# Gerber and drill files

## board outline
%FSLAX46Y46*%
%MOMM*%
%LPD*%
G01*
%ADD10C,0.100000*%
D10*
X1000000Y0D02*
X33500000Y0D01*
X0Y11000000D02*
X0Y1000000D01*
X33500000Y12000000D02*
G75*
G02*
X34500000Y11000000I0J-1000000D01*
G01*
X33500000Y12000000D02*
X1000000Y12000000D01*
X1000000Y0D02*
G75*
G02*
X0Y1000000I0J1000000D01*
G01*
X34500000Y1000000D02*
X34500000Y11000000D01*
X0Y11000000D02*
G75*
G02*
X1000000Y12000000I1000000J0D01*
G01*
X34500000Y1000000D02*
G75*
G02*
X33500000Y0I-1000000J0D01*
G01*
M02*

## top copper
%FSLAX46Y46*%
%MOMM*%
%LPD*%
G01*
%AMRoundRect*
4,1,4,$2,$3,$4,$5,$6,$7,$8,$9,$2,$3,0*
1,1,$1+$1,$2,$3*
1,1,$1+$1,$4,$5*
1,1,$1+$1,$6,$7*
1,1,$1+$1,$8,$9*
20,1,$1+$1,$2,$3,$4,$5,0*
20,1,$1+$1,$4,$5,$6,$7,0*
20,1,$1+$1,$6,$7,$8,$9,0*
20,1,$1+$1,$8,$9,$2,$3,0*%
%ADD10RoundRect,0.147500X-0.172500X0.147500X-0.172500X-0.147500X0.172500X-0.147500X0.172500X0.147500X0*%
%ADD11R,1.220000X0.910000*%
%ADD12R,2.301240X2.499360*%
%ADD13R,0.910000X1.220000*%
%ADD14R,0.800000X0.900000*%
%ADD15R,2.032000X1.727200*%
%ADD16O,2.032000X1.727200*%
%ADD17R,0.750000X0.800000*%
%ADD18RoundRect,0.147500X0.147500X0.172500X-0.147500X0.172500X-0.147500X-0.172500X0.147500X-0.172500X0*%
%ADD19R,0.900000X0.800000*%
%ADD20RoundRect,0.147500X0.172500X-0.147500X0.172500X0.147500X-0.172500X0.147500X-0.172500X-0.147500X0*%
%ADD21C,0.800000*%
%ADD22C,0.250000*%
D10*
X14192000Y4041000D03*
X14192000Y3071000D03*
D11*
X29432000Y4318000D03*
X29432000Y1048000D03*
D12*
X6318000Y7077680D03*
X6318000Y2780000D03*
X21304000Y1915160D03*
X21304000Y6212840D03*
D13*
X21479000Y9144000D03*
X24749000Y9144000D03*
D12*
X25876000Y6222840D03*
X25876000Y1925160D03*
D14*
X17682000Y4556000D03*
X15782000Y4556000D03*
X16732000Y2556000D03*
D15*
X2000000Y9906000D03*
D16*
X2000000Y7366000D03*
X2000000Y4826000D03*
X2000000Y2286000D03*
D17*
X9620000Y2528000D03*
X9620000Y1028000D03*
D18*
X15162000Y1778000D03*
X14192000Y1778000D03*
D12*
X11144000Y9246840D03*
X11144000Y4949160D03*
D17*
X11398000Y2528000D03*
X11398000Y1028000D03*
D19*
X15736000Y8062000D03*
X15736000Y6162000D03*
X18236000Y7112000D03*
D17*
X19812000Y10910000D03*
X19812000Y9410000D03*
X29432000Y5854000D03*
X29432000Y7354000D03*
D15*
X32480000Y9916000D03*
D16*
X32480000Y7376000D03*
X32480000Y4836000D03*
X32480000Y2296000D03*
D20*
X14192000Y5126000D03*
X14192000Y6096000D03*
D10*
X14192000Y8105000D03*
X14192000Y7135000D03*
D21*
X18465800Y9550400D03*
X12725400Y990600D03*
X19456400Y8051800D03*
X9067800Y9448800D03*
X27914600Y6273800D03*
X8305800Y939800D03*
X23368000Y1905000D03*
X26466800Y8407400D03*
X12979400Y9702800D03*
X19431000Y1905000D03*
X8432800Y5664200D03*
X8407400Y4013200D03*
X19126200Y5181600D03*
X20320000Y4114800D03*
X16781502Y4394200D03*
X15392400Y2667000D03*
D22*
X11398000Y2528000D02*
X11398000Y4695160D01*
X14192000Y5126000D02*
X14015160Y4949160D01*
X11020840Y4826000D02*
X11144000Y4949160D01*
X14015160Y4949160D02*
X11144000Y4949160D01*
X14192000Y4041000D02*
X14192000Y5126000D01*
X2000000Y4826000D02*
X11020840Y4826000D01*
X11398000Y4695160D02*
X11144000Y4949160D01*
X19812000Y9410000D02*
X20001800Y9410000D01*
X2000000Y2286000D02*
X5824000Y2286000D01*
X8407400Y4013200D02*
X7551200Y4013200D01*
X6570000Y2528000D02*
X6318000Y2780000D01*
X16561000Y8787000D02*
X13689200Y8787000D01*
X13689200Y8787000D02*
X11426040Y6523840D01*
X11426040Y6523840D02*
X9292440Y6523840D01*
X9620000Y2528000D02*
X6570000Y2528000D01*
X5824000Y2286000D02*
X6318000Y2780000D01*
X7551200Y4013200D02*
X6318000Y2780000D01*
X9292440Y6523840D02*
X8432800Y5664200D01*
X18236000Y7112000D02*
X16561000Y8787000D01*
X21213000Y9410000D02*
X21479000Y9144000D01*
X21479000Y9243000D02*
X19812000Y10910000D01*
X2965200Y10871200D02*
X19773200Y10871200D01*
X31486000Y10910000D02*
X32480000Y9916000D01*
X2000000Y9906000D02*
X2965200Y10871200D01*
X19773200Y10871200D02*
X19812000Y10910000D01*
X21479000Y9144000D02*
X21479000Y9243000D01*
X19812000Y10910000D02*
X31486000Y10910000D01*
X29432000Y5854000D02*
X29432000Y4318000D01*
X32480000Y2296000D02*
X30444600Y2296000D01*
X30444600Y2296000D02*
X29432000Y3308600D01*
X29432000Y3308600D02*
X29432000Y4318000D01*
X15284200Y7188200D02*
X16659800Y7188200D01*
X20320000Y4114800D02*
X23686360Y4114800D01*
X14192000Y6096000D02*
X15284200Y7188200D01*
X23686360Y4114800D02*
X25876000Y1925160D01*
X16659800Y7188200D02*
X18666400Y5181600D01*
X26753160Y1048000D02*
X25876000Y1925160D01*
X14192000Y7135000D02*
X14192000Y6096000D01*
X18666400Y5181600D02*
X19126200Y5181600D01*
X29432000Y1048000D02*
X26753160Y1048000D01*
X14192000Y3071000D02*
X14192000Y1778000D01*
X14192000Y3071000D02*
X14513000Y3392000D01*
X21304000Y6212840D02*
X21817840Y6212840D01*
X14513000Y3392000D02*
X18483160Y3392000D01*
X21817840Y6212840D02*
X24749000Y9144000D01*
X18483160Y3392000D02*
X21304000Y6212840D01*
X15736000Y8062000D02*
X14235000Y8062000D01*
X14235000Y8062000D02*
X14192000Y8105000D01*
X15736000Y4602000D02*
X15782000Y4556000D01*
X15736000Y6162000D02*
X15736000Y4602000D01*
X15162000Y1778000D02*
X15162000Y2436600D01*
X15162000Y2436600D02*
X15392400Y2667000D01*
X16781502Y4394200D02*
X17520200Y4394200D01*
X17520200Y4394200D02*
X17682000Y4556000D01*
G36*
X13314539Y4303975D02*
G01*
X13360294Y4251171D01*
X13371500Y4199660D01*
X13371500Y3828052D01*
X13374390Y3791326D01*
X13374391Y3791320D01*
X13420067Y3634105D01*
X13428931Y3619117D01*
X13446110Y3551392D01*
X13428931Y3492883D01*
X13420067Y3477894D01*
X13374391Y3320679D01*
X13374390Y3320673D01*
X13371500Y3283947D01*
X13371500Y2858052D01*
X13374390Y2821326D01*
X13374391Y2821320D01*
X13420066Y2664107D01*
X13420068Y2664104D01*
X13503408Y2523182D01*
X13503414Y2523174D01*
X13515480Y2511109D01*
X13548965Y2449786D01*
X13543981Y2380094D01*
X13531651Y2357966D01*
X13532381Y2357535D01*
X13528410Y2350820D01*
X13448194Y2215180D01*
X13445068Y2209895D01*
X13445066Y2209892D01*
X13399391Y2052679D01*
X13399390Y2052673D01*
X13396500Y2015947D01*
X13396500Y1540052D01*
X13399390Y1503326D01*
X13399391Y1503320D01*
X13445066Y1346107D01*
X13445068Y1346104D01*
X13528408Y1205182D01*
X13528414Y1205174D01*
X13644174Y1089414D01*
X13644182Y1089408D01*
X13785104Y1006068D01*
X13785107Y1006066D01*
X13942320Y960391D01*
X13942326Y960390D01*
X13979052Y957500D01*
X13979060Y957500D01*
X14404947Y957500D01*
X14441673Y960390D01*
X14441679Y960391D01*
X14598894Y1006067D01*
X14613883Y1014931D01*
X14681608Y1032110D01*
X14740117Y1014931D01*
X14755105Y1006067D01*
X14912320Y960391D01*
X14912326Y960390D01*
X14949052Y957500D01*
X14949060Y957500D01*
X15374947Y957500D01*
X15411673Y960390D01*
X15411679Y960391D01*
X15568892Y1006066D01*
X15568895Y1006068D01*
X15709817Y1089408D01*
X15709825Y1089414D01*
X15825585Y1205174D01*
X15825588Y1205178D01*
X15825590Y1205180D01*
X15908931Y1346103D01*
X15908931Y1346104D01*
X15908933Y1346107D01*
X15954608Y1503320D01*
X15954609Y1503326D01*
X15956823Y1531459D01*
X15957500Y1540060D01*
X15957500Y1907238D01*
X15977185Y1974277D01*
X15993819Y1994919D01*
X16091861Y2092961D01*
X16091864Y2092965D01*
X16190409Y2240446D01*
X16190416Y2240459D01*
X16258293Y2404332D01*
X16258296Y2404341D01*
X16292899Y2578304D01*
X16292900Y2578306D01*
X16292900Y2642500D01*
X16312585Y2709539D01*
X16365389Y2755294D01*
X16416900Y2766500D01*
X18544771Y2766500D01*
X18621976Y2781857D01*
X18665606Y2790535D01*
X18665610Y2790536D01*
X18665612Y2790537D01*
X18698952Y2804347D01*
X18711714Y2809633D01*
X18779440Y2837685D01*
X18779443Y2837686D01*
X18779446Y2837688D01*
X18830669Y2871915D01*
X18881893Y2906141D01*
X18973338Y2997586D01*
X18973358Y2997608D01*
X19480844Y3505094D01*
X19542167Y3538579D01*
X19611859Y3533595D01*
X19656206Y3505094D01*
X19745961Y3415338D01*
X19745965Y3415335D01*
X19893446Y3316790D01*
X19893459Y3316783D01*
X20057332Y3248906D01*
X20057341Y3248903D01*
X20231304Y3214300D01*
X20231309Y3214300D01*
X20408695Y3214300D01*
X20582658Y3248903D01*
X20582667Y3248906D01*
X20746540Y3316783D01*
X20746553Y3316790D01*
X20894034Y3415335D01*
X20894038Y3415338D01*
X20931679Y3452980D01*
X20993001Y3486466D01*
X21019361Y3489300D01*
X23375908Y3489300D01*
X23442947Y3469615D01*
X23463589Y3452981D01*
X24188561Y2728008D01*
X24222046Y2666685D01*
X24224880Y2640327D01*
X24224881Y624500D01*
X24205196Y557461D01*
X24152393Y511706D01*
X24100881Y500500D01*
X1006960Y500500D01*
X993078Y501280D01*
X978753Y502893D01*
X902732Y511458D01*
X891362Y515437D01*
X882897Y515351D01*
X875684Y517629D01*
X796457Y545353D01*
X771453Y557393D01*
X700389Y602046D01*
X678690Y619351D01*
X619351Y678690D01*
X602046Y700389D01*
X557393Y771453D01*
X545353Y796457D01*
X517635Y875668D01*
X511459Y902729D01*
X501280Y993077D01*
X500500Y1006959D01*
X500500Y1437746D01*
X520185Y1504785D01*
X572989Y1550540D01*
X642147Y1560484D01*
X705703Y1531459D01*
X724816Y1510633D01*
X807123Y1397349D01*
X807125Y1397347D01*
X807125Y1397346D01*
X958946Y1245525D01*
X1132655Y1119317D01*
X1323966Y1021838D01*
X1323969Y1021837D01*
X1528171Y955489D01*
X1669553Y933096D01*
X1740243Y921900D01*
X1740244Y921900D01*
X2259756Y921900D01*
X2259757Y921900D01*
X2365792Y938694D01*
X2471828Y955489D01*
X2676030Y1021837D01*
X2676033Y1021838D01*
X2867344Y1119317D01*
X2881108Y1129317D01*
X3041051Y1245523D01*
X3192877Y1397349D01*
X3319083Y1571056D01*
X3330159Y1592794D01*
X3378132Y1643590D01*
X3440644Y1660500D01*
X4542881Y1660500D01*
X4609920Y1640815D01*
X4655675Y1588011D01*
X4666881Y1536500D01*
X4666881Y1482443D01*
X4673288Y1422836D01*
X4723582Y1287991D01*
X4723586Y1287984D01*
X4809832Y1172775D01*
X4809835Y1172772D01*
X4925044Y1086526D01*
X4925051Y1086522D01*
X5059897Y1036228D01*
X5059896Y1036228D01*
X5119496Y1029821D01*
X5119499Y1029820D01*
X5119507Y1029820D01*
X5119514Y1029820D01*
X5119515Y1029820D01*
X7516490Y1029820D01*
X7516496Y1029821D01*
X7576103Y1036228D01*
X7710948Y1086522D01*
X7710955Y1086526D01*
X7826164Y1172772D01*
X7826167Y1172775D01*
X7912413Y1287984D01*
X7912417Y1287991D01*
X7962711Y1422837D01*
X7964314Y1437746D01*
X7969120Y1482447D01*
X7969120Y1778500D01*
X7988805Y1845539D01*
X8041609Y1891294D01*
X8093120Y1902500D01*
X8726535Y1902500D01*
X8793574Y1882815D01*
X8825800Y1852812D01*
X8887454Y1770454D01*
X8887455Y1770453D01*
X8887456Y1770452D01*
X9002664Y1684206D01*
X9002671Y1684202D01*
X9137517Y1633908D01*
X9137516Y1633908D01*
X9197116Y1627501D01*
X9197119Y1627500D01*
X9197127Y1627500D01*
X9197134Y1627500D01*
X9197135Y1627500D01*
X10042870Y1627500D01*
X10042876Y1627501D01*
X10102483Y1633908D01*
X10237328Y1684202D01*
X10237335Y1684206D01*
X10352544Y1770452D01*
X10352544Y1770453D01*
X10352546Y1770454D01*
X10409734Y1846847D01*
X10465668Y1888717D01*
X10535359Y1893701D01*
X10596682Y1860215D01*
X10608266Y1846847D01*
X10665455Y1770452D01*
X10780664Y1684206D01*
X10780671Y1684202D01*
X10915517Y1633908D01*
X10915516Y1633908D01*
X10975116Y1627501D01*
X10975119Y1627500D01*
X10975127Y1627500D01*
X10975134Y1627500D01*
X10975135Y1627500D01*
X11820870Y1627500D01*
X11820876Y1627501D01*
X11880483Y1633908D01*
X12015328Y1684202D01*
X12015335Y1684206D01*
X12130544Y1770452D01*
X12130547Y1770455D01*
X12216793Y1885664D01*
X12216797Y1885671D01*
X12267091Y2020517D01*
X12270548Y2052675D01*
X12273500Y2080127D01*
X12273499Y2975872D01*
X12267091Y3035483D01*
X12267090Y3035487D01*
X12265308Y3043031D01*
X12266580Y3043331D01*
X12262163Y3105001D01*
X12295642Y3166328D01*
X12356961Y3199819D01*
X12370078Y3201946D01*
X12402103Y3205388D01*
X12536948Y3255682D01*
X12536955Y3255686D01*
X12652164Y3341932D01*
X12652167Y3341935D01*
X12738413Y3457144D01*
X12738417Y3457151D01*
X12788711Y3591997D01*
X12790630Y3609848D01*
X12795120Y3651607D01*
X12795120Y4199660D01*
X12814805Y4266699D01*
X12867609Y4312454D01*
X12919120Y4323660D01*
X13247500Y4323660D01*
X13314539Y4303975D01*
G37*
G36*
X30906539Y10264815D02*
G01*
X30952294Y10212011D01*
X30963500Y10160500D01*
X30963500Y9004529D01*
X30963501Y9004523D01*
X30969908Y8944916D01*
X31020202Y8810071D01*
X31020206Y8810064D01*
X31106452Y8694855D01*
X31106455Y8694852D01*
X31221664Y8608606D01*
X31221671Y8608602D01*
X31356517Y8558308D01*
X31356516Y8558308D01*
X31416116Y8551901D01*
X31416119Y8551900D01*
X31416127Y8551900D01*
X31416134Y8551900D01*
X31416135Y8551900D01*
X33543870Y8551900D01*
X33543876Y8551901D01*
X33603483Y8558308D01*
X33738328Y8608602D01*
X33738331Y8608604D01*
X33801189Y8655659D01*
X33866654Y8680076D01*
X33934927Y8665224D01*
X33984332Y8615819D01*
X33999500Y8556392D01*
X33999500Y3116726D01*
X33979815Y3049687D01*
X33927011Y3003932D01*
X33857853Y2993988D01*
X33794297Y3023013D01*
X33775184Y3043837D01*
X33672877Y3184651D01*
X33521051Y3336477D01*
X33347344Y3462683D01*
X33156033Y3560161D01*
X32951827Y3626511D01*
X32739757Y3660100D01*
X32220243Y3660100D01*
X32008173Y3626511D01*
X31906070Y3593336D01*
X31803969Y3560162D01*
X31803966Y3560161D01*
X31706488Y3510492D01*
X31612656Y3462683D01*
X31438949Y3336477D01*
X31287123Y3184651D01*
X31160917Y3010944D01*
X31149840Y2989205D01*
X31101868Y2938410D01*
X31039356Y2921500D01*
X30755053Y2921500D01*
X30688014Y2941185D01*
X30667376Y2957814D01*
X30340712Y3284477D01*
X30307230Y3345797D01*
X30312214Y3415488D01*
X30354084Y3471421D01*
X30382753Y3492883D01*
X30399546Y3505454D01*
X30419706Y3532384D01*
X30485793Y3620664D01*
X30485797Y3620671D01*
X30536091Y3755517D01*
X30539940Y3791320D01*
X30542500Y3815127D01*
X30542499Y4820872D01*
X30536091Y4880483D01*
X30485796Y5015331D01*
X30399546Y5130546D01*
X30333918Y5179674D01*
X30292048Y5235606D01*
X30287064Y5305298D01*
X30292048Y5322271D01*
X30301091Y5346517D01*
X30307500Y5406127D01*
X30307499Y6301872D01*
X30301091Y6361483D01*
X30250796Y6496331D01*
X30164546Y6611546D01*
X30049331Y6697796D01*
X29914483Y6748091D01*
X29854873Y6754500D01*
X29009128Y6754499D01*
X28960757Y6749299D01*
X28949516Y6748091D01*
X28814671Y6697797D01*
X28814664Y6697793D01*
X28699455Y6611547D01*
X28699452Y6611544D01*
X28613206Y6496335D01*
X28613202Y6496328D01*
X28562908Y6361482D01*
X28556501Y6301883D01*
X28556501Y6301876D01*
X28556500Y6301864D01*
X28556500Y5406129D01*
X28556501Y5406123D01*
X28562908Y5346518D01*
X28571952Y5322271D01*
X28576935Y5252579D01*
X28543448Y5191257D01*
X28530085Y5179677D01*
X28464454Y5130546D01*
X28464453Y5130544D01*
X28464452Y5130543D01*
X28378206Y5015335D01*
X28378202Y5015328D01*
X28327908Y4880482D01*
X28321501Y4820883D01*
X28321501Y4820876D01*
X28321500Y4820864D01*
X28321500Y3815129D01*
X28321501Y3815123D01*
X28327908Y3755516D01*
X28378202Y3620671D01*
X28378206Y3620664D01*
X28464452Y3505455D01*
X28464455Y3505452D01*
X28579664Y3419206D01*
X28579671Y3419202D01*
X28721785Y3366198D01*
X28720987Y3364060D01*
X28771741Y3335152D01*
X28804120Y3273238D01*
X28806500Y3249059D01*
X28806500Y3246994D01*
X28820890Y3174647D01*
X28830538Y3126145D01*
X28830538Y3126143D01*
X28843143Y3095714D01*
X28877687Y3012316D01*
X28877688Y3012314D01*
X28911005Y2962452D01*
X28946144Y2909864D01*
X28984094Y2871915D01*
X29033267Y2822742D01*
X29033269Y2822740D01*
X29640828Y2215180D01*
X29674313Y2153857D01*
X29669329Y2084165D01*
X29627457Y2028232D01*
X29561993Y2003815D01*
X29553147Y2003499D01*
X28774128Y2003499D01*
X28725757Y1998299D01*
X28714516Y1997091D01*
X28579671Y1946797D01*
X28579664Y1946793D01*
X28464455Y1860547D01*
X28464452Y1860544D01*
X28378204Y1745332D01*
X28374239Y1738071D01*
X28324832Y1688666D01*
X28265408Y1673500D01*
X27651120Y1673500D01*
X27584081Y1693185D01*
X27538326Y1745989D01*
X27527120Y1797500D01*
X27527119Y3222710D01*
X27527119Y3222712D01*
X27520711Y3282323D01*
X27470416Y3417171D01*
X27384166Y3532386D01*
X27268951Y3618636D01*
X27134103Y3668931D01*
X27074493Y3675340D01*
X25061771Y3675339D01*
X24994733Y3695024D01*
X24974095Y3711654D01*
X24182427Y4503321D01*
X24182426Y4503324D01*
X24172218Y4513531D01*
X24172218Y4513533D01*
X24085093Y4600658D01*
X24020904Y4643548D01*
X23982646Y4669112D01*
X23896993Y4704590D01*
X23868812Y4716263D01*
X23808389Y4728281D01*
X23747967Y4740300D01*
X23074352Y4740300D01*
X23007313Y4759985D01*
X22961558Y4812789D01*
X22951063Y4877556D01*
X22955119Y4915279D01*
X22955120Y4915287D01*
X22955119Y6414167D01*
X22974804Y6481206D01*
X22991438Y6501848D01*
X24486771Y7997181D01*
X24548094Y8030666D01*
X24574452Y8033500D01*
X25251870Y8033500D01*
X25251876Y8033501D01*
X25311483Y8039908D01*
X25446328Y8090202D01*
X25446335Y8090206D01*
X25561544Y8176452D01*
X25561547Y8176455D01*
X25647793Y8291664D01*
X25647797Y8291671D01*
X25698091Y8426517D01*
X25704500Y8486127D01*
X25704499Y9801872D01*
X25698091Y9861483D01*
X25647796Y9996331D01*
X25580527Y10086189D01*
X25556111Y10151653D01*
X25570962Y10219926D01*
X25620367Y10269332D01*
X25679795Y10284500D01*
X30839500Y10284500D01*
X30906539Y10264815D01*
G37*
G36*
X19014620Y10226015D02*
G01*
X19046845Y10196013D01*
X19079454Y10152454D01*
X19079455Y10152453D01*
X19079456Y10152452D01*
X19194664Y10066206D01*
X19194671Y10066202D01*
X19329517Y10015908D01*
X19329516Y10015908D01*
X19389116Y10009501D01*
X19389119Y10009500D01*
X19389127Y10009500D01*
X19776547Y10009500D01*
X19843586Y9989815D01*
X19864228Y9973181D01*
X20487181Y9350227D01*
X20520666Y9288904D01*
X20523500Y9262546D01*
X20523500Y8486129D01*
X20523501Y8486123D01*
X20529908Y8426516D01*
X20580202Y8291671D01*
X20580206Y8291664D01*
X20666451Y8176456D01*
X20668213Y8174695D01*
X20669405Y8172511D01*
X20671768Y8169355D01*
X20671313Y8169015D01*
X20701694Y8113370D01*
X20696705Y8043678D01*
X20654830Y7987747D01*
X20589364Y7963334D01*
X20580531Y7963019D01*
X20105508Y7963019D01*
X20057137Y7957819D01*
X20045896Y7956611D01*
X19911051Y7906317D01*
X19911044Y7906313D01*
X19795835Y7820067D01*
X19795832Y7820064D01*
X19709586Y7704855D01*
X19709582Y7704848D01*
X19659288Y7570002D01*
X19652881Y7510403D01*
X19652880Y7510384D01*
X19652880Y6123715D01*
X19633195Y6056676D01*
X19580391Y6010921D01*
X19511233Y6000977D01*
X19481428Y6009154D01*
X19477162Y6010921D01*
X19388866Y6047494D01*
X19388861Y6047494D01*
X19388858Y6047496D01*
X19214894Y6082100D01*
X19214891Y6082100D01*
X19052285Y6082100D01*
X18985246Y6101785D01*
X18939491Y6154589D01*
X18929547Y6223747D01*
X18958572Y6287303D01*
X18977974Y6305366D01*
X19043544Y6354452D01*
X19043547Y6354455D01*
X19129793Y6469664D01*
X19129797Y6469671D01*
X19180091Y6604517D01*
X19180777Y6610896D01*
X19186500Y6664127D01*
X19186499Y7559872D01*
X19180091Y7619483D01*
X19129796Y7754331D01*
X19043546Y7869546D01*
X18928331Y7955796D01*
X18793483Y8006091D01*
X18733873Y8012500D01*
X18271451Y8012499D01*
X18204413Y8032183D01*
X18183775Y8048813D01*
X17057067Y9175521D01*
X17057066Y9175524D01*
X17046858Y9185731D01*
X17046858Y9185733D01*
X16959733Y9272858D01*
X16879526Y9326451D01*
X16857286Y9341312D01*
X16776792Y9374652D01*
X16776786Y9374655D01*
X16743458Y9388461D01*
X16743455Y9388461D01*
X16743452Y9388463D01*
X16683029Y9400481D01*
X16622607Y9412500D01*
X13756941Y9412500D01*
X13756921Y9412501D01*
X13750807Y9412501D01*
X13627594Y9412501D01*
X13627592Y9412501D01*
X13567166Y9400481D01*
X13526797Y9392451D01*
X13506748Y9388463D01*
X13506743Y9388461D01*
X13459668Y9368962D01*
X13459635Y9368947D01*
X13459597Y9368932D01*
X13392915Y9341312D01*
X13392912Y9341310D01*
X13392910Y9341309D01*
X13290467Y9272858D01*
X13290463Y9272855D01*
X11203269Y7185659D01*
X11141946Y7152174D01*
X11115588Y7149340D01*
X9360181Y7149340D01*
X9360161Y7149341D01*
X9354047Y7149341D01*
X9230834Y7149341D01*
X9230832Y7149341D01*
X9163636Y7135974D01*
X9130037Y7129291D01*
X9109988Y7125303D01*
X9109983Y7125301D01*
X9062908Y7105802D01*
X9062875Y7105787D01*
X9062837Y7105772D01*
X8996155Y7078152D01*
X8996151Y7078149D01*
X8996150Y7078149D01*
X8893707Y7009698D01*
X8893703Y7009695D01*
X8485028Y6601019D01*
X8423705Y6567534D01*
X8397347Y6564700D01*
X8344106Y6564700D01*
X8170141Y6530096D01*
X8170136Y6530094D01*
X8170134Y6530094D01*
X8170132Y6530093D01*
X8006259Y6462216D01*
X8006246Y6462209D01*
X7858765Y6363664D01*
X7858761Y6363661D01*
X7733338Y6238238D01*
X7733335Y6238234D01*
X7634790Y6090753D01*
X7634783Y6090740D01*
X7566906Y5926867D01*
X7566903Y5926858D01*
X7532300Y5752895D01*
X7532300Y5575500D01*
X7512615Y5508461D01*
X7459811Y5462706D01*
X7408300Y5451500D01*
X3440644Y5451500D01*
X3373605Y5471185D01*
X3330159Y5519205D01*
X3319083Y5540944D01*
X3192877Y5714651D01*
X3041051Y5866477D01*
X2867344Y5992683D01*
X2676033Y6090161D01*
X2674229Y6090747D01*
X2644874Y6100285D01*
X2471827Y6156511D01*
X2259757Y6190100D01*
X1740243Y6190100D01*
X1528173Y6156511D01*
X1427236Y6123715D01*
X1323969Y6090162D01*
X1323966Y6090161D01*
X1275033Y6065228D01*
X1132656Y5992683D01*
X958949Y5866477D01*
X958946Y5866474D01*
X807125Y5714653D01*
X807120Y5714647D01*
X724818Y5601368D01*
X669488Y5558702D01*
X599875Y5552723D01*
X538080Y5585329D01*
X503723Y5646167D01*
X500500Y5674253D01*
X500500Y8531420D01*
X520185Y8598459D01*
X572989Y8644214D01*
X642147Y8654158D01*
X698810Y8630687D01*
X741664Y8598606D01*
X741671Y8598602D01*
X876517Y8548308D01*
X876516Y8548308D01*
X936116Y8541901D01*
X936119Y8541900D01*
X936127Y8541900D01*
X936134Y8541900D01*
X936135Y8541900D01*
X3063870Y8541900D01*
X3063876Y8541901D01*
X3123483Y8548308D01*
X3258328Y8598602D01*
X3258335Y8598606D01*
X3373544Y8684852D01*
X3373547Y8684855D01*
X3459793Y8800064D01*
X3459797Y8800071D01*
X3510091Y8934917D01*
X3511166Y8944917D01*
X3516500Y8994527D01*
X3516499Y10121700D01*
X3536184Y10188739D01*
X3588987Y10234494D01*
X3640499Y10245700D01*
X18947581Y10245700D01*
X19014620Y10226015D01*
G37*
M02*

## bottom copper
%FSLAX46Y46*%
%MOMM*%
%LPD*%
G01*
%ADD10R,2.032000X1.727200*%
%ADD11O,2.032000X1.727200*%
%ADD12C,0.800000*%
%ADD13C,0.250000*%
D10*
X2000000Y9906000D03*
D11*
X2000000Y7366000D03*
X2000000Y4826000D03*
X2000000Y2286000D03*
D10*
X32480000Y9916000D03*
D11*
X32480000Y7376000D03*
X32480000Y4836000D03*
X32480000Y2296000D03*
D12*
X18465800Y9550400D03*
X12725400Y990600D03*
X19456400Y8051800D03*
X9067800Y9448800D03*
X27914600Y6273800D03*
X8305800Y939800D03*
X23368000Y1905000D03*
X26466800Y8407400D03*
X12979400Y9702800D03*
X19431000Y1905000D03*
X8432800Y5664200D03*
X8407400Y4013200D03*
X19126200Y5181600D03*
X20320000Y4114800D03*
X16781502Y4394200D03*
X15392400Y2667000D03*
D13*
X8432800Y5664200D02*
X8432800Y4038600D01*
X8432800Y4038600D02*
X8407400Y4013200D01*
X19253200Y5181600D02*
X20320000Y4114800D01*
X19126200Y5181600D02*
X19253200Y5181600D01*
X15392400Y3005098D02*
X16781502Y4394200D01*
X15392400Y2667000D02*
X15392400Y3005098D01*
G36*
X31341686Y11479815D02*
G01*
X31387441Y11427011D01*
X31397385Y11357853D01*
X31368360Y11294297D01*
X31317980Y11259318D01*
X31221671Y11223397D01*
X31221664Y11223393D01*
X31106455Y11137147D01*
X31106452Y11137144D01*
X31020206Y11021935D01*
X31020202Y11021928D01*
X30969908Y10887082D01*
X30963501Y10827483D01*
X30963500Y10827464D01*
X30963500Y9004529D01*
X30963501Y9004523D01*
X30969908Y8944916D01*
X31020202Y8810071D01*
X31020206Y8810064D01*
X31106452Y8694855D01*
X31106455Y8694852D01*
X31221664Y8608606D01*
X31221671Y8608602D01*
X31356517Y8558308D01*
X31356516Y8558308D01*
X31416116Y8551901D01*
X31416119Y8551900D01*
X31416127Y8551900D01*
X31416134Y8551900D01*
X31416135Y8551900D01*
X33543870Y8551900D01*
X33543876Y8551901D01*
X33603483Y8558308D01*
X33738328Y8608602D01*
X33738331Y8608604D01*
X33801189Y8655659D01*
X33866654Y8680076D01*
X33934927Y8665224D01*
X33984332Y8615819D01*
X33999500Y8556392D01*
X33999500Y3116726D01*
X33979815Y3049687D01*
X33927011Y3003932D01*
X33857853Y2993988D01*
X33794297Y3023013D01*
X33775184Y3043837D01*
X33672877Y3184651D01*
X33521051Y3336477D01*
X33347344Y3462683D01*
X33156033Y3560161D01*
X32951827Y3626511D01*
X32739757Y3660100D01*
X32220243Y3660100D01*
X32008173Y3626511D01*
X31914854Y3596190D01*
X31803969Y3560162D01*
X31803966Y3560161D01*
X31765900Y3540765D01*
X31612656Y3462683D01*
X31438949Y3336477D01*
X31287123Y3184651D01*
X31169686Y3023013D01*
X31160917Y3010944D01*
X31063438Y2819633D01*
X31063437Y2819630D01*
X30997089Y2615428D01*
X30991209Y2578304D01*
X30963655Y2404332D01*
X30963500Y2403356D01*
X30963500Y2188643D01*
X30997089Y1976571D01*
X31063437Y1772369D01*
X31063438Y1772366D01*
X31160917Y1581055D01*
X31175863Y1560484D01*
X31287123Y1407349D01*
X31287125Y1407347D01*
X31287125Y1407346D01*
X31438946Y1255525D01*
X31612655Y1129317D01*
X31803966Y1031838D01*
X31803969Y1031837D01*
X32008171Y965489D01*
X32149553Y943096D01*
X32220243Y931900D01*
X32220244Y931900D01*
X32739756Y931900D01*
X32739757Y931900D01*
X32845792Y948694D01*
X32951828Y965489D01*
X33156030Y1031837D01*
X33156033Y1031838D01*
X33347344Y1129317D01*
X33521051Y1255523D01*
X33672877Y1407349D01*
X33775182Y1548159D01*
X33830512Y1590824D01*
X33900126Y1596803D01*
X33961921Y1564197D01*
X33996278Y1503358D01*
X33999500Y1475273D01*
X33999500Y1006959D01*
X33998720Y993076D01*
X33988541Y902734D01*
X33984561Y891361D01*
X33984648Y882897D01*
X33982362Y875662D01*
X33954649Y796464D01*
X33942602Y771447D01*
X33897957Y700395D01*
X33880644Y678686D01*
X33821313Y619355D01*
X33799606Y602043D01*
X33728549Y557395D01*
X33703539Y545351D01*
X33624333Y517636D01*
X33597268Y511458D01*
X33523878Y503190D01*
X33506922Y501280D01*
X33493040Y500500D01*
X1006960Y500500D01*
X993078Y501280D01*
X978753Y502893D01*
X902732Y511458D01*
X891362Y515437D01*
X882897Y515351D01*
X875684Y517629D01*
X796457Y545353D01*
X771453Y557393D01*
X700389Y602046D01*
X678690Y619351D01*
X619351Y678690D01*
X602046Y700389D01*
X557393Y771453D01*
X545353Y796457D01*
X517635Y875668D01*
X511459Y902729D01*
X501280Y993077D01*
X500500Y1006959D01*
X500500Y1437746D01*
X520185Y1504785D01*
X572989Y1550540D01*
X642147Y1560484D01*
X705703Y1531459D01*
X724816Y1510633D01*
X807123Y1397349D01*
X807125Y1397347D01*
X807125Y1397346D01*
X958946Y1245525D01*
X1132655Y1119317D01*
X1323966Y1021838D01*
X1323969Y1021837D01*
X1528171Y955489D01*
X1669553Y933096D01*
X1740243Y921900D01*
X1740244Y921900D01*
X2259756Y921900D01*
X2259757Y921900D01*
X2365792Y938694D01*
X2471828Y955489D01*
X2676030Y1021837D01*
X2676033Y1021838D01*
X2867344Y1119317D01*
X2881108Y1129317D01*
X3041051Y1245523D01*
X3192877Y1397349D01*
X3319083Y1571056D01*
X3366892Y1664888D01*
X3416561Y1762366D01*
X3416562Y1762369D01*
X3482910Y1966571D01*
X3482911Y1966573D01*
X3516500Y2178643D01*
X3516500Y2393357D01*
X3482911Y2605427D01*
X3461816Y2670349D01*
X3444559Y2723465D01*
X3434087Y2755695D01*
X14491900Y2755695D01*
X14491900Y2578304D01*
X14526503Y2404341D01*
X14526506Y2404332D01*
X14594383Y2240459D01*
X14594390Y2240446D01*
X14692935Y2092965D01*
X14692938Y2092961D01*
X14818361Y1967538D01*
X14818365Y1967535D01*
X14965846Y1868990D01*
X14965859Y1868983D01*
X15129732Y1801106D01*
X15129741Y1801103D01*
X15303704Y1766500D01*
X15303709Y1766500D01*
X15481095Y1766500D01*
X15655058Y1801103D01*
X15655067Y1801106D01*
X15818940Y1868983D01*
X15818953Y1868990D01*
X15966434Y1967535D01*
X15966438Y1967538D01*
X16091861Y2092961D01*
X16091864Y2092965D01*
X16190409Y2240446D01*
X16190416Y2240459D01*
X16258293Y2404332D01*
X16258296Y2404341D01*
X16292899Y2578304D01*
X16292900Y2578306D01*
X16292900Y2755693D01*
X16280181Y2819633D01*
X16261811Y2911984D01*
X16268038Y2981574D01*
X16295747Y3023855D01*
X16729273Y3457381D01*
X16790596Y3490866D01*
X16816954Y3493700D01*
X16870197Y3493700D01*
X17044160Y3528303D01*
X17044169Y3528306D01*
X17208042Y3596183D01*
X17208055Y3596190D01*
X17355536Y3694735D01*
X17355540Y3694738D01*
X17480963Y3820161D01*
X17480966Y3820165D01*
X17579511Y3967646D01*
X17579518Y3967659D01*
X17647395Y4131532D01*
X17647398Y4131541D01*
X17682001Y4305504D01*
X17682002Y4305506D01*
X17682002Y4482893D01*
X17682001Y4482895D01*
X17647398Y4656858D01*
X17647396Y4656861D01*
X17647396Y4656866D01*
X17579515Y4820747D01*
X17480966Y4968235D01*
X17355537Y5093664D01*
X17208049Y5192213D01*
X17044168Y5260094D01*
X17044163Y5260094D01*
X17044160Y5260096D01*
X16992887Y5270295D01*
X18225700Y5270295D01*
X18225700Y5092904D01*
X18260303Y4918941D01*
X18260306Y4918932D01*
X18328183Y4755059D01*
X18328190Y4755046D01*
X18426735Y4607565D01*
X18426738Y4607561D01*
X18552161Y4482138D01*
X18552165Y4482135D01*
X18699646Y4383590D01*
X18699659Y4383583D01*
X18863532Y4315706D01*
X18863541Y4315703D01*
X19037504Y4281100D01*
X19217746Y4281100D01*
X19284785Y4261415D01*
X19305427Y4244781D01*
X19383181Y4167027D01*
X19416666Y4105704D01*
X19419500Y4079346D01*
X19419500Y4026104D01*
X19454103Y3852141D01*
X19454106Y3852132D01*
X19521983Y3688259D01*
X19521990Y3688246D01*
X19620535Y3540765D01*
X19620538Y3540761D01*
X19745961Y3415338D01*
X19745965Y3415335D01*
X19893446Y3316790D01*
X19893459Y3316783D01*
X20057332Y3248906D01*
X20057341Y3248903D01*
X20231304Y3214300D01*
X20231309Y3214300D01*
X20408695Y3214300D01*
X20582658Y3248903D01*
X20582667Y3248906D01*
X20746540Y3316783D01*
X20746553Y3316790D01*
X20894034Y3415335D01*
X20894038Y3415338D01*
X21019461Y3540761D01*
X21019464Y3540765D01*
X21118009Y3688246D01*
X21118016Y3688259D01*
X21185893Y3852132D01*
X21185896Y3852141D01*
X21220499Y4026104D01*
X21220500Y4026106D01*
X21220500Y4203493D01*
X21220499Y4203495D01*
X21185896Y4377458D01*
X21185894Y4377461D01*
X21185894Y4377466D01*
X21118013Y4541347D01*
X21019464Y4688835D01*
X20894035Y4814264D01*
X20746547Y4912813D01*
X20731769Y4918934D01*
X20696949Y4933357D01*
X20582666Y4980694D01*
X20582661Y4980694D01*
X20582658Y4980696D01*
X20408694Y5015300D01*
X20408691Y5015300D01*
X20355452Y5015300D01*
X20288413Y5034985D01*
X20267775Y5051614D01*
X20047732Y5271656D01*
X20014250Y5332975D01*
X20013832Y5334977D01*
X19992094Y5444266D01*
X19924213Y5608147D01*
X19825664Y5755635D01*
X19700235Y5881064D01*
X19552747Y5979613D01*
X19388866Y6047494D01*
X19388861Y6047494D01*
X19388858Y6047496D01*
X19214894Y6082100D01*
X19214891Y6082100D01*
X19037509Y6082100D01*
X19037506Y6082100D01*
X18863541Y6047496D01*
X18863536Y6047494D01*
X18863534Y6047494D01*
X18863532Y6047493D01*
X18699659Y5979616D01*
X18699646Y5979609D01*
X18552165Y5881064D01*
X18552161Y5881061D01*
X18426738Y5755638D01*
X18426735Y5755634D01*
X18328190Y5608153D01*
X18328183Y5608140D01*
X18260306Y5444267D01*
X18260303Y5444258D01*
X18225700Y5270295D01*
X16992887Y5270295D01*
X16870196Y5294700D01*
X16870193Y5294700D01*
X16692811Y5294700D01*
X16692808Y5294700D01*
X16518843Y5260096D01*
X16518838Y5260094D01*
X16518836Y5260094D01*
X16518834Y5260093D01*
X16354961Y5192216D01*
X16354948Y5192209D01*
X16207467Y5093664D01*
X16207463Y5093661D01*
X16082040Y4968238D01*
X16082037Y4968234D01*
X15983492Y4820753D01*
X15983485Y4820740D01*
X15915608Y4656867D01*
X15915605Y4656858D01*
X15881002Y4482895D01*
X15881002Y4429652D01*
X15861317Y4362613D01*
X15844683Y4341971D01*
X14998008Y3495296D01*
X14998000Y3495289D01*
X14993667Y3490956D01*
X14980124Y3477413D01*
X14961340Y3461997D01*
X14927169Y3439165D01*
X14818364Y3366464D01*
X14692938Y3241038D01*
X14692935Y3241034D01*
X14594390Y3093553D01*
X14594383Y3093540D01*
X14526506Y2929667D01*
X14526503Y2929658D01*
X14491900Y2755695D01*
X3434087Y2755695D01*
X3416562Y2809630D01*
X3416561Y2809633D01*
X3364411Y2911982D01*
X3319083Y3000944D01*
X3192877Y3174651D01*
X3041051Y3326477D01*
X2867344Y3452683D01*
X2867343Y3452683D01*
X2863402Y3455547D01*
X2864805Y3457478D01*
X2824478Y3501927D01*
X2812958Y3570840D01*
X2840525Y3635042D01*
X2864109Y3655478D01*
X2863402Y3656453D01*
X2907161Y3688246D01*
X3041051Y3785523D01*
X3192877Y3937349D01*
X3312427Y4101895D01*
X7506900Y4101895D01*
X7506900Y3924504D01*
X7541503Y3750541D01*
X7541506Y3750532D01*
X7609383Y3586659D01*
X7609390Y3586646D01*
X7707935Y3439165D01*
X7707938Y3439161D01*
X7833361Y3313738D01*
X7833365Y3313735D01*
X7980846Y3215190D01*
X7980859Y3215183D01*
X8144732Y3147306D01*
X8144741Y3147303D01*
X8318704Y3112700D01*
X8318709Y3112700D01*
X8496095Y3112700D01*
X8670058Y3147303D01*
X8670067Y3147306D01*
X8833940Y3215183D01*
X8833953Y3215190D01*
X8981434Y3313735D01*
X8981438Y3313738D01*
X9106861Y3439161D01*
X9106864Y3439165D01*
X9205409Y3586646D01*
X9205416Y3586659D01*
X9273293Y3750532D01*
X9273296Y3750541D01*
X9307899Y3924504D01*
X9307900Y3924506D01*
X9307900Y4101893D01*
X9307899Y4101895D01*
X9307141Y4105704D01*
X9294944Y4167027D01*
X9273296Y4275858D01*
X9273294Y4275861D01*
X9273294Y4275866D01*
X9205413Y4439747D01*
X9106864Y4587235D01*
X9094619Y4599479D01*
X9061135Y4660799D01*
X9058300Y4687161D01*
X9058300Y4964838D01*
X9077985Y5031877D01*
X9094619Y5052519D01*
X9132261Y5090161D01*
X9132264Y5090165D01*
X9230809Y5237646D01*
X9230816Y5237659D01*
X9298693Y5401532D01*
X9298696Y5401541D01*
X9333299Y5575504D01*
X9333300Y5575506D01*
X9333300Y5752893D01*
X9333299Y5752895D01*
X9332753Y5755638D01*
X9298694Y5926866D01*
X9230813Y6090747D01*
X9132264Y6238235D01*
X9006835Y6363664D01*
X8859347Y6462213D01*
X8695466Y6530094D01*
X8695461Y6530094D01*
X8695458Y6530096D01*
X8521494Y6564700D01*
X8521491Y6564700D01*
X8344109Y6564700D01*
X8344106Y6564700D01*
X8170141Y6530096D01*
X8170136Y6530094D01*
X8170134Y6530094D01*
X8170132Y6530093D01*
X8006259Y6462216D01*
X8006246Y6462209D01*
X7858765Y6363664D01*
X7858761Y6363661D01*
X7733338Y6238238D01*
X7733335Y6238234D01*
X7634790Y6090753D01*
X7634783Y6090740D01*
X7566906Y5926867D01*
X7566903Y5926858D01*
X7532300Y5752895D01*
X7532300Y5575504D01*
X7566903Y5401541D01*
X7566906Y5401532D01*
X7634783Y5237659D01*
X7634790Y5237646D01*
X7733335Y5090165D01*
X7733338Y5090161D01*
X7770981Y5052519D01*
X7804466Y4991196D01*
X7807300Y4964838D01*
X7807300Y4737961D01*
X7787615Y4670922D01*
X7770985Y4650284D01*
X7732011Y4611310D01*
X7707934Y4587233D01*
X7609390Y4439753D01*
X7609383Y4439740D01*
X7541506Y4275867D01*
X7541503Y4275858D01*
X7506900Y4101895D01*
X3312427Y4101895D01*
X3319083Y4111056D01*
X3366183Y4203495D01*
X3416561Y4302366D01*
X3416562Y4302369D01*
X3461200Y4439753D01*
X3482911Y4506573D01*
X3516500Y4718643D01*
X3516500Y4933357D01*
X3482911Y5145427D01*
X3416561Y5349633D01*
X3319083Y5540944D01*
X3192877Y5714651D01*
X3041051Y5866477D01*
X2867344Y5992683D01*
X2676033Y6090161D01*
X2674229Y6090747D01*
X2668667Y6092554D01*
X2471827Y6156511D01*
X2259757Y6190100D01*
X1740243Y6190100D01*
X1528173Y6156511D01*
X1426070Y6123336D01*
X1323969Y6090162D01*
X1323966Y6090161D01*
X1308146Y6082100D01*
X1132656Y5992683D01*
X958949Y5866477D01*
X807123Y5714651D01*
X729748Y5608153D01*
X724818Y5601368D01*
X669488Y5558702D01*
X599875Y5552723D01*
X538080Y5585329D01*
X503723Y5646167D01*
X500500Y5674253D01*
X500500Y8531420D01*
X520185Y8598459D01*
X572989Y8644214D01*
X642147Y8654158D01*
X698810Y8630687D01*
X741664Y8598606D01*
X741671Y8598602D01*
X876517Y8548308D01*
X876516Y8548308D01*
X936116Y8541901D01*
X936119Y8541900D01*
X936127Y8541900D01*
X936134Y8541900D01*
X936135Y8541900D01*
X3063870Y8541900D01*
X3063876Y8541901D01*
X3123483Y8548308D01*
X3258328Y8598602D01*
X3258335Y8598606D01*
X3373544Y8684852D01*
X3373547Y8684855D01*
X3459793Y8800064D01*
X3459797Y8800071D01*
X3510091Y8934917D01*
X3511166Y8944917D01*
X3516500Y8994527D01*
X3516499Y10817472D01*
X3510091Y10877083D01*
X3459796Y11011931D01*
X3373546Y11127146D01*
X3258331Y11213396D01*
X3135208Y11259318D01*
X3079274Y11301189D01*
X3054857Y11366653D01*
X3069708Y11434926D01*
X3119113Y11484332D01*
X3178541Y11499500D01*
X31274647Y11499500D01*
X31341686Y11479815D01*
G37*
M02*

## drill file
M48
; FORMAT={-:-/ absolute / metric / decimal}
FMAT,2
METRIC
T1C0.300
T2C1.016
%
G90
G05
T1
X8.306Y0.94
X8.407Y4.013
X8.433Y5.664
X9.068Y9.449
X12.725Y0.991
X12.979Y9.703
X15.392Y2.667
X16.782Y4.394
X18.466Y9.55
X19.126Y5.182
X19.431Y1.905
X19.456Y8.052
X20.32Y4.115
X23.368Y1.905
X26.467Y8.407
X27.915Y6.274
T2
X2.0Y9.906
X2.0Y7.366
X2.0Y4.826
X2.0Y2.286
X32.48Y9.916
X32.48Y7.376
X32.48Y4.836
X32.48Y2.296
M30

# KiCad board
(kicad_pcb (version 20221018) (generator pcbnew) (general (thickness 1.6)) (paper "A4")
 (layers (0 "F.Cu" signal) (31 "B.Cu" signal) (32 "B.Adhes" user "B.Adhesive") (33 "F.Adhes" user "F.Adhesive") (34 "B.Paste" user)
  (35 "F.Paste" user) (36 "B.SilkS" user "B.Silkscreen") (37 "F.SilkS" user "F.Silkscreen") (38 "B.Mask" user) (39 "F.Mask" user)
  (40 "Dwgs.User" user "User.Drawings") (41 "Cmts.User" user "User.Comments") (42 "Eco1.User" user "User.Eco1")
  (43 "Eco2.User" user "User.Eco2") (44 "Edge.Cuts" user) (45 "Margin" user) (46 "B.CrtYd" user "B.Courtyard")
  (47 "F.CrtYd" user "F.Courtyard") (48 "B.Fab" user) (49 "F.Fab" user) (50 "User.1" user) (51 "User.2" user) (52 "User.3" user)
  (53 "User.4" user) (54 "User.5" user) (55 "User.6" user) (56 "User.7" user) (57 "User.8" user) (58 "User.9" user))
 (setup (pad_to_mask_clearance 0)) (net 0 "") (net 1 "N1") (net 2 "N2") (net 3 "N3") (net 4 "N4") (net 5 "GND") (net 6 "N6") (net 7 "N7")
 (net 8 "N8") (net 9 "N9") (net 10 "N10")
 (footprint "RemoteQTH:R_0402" (layer "F.Cu") (at 14.192 -3.556 -90)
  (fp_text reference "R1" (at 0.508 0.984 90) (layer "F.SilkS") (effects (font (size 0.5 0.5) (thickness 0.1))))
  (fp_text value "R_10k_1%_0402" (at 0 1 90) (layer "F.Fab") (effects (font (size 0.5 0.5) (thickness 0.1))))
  (pad "1" smd roundrect (at -0.485 0 270) (size 0.59 0.64) (layers "F.Cu" "F.Paste" "F.Mask") (roundrect_rratio 0.25) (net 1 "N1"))
  (pad "2" smd roundrect (at 0.485 0 270) (size 0.59 0.64) (layers "F.Cu" "F.Paste" "F.Mask") (roundrect_rratio 0.25) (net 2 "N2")))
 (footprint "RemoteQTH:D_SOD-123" (layer "F.Cu") (at 29.432 -2.683 -90)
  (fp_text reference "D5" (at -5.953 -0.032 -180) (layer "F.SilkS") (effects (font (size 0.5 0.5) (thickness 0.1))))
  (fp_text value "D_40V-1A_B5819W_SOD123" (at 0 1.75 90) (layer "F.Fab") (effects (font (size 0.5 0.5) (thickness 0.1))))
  (pad "1" smd rect (at -1.635 0 270) (size 0.91 1.22) (layers "F.Cu" "F.Paste" "F.Mask") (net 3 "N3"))
  (pad "2" smd rect (at 1.635 0 270) (size 0.91 1.22) (layers "F.Cu" "F.Paste" "F.Mask") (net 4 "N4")))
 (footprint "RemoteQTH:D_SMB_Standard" (layer "F.Cu") (at 6.318 -4.92884 -90)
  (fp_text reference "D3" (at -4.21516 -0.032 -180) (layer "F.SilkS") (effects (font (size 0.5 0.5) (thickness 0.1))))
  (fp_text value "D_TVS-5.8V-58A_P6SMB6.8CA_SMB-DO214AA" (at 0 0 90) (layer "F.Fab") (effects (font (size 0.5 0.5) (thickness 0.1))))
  (pad "1" smd rect (at -2.14884 0 270) (size 2.49936 2.30124) (layers "F.Cu" "F.Paste" "F.Mask") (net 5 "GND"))
  (pad "2" smd rect (at 2.14884 0 270) (size 2.49936 2.30124) (layers "F.Cu" "F.Paste" "F.Mask") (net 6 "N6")))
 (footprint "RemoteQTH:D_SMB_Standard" (layer "F.Cu") (at 21.304 -4.064 90)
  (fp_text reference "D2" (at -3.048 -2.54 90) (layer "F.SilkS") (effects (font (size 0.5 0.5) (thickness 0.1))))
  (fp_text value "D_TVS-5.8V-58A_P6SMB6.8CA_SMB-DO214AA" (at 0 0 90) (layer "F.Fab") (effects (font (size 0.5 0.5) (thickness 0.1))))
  (pad "1" smd rect (at -2.14884 0 90) (size 2.49936 2.30124) (layers "F.Cu" "F.Paste" "F.Mask") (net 5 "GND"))
  (pad "2" smd rect (at 2.14884 0 90) (size 2.49936 2.30124) (layers "F.Cu" "F.Paste" "F.Mask") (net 2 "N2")))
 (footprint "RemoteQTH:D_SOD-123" (layer "F.Cu") (at 23.114 -9.144)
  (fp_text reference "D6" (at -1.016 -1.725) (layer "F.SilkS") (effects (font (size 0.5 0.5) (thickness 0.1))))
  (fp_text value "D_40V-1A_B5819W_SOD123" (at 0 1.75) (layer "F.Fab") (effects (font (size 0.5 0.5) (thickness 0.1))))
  (pad "1" smd rect (at -1.635 0) (size 0.91 1.22) (layers "F.Cu" "F.Paste" "F.Mask") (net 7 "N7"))
  (pad "2" smd rect (at 1.635 0) (size 0.91 1.22) (layers "F.Cu" "F.Paste" "F.Mask") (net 2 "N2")))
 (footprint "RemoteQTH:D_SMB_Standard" (layer "F.Cu") (at 25.876 -4.074 -90)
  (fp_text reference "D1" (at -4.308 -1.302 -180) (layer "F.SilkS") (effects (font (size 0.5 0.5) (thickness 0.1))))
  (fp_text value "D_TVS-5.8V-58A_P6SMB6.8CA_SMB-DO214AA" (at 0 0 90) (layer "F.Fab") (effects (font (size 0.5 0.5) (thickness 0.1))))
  (pad "1" smd rect (at -2.14884 0 270) (size 2.49936 2.30124) (layers "F.Cu" "F.Paste" "F.Mask") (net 5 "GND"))
  (pad "2" smd rect (at 2.14884 0 270) (size 2.49936 2.30124) (layers "F.Cu" "F.Paste" "F.Mask") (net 4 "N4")))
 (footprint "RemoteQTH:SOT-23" (layer "F.Cu") (at 16.732 -3.556 90)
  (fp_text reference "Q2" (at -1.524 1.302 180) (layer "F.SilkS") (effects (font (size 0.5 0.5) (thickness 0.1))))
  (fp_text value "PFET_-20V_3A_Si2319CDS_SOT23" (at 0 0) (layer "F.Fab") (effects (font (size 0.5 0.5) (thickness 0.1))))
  (pad "1" smd rect (at 1 0.95 270) (size 0.9 0.8) (layers "F.Cu" "F.Paste" "F.Mask") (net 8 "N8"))
  (pad "2" smd rect (at 1 -0.95 270) (size 0.9 0.8) (layers "F.Cu" "F.Paste" "F.Mask") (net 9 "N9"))
  (pad "3" smd rect (at -1 0 270) (size 0.9 0.8) (layers "F.Cu" "F.Paste" "F.Mask") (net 5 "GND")))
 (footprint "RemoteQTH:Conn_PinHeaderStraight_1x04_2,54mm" (layer "F.Cu") (at 2 -9.906)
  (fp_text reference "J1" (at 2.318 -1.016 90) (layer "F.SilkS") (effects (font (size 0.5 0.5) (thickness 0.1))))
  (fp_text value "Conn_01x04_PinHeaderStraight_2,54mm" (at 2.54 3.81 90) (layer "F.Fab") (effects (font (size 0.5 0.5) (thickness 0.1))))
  (pad "1" thru_hole rect (at 0 0) (size 2.032 1.7272) (drill 1.016) (layers "*.Cu" "*.Mask") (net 7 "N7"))
  (pad "2" thru_hole oval (at 0 2.54) (size 2.032 1.7272) (drill 1.016) (layers "*.Cu" "*.Mask") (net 5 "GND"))
  (pad "3" thru_hole oval (at 0 5.08) (size 2.032 1.7272) (drill 1.016) (layers "*.Cu" "*.Mask") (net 1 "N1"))
  (pad "4" thru_hole oval (at 0 7.62) (size 2.032 1.7272) (drill 1.016) (layers "*.Cu" "*.Mask") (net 6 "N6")))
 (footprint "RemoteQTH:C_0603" (layer "F.Cu") (at 9.62 -1.778 -90)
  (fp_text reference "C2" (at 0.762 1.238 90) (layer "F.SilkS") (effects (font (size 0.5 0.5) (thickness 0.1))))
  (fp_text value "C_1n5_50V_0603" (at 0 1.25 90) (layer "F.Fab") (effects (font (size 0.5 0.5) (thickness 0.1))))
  (pad "1" smd rect (at -0.75 0 270) (size 0.8 0.75) (layers "F.Cu" "F.Paste" "F.Mask") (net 6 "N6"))
  (pad "2" smd rect (at 0.75 0 270) (size 0.8 0.75) (layers "F.Cu" "F.Paste" "F.Mask") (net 5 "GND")))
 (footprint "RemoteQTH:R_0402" (layer "F.Cu") (at 14.677 -1.778 180)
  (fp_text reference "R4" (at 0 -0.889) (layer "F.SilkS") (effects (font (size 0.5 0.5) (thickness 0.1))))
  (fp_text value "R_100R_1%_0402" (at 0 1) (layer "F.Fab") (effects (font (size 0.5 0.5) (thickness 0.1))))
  (pad "1" smd roundrect (at -0.485 0 180) (size 0.59 0.64) (layers "F.Cu" "F.Paste" "F.Mask") (roundrect_rratio 0.25) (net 8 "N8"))
  (pad "2" smd roundrect (at 0.485 0 180) (size 0.59 0.64) (layers "F.Cu" "F.Paste" "F.Mask") (roundrect_rratio 0.25) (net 2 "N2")))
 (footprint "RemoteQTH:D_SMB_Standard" (layer "F.Cu") (at 11.144 -7.098 -90)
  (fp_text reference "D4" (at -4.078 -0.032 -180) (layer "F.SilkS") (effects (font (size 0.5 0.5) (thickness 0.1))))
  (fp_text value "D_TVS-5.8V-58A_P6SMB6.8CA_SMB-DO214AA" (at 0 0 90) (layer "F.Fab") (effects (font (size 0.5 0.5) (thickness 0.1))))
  (pad "1" smd rect (at -2.14884 0 270) (size 2.49936 2.30124) (layers "F.Cu" "F.Paste" "F.Mask") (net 5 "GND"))
  (pad "2" smd rect (at 2.14884 0 270) (size 2.49936 2.30124) (layers "F.Cu" "F.Paste" "F.Mask") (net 1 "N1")))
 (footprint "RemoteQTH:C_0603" (layer "F.Cu") (at 11.398 -1.778 -90)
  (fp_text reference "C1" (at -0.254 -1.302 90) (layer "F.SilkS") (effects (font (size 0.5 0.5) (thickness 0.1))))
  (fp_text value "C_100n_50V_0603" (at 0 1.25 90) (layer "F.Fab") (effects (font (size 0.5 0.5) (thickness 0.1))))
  (pad "1" smd rect (at -0.75 0 270) (size 0.8 0.75) (layers "F.Cu" "F.Paste" "F.Mask") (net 1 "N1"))
  (pad "2" smd rect (at 0.75 0 270) (size 0.8 0.75) (layers "F.Cu" "F.Paste" "F.Mask") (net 5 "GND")))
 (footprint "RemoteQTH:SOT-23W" (layer "F.Cu") (at 16.986 -7.112 180)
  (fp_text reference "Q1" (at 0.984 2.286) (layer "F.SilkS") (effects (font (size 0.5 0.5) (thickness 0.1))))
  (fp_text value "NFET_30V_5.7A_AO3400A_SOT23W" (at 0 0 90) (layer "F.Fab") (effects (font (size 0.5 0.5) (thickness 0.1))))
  (pad "1" smd rect (at 1.25 0.95) (size 0.9 0.8) (layers "F.Cu" "F.Paste" "F.Mask") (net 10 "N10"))
  (pad "2" smd rect (at 1.25 -0.95) (size 0.9 0.8) (layers "F.Cu" "F.Paste" "F.Mask") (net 9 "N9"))
  (pad "3" smd rect (at -1.25 0) (size 0.9 0.8) (layers "F.Cu" "F.Paste" "F.Mask") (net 6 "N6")))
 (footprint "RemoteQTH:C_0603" (layer "F.Cu") (at 19.812 -10.16 -90)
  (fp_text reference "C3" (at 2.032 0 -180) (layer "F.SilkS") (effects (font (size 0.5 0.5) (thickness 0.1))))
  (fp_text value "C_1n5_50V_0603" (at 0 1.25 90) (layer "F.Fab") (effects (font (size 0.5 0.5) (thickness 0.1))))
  (pad "1" smd rect (at -0.75 0 270) (size 0.8 0.75) (layers "F.Cu" "F.Paste" "F.Mask") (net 7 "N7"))
  (pad "2" smd rect (at 0.75 0 270) (size 0.8 0.75) (layers "F.Cu" "F.Paste" "F.Mask") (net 5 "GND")))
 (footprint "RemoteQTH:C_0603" (layer "F.Cu") (at 29.432 -6.604 90)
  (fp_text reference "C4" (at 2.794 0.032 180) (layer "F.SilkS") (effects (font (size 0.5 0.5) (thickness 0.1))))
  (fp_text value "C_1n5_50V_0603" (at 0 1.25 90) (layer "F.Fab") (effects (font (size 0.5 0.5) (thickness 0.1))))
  (pad "1" smd rect (at -0.75 0 90) (size 0.8 0.75) (layers "F.Cu" "F.Paste" "F.Mask") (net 3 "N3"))
  (pad "2" smd rect (at 0.75 0 90) (size 0.8 0.75) (layers "F.Cu" "F.Paste" "F.Mask") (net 5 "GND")))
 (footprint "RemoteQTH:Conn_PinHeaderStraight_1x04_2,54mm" (layer "F.Cu") (at 32.48 -9.916)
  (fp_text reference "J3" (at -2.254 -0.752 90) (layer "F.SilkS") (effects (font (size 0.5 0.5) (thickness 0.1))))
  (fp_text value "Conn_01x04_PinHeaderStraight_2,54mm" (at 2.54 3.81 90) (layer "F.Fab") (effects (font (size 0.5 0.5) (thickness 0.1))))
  (pad "1" thru_hole rect (at 0 0) (size 2.032 1.7272) (drill 1.016) (layers "*.Cu" "*.Mask") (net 7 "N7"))
  (pad "2" thru_hole oval (at 0 2.54) (size 2.032 1.7272) (drill 1.016) (layers "*.Cu" "*.Mask") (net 5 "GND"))
  (pad "3" thru_hole oval (at 0 5.08) (size 2.032 1.7272) (drill 1.016) (layers "*.Cu" "*.Mask") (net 5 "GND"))
  (pad "4" thru_hole oval (at 0 7.62) (size 2.032 1.7272) (drill 1.016) (layers "*.Cu" "*.Mask") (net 3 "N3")))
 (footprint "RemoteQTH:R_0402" (layer "F.Cu") (at 14.192 -5.611 90)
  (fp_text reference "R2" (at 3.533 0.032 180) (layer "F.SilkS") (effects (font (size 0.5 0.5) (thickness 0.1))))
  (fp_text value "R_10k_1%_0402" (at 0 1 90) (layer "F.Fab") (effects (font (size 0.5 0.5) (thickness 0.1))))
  (pad "1" smd roundrect (at -0.485 0 90) (size 0.59 0.64) (layers "F.Cu" "F.Paste" "F.Mask") (roundrect_rratio 0.25) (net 1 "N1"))
  (pad "2" smd roundrect (at 0.485 0 90) (size 0.59 0.64) (layers "F.Cu" "F.Paste" "F.Mask") (roundrect_rratio 0.25) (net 4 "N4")))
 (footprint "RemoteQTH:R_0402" (layer "F.Cu") (at 14.192 -7.62 -90)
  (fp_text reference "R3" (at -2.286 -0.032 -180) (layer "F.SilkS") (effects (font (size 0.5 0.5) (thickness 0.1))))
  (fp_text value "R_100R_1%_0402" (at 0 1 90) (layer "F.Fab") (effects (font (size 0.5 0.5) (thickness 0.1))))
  (pad "1" smd roundrect (at -0.485 0 270) (size 0.59 0.64) (layers "F.Cu" "F.Paste" "F.Mask") (roundrect_rratio 0.25) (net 10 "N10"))
  (pad "2" smd roundrect (at 0.485 0 270) (size 0.59 0.64) (layers "F.Cu" "F.Paste" "F.Mask") (roundrect_rratio 0.25) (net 4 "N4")))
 (gr_line (start 1 0) (end 33.5 0) (stroke (width 0.1) (type default)) (layer "Edge.Cuts"))
 (gr_line (start 0 -11) (end 0 -1) (stroke (width 0.1) (type default)) (layer "Edge.Cuts"))
 (gr_arc (start 33.5 -12) (mid 34.207107 -11.707107) (end 34.5 -11) (stroke (width 0.1) (type default)) (layer "Edge.Cuts"))
 (gr_line (start 33.5 -12) (end 1 -12) (stroke (width 0.1) (type default)) (layer "Edge.Cuts"))
 (gr_arc (start 1 0) (mid 0.292893 -0.292893) (end 0 -1) (stroke (width 0.1) (type default)) (layer "Edge.Cuts"))
 (gr_line (start 34.5 -1) (end 34.5 -11) (stroke (width 0.1) (type default)) (layer "Edge.Cuts"))
 (gr_arc (start 0 -11) (mid 0.292893 -11.707107) (end 1 -12) (stroke (width 0.1) (type default)) (layer "Edge.Cuts"))
 (gr_arc (start 34.5 -1) (mid 34.207107 -0.292893) (end 33.5 0) (stroke (width 0.1) (type default)) (layer "Edge.Cuts"))
 (segment (start 11.398 -2.528) (end 11.398 -4.69516) (width 0.25) (layer "F.Cu") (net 1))
 (segment (start 14.192 -5.126) (end 14.01516 -4.94916) (width 0.25) (layer "F.Cu") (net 1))
 (segment (start 11.02084 -4.826) (end 11.144 -4.94916) (width 0.25) (layer "F.Cu") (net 1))
 (segment (start 14.01516 -4.94916) (end 11.144 -4.94916) (width 0.25) (layer "F.Cu") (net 1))
 (segment (start 14.192 -4.041) (end 14.192 -5.126) (width 0.25) (layer "F.Cu") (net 1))
 (segment (start 2 -4.826) (end 11.02084 -4.826) (width 0.25) (layer "F.Cu") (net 1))
 (segment (start 11.398 -4.69516) (end 11.144 -4.94916) (width 0.25) (layer "F.Cu") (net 1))
 (segment (start 19.812 -9.41) (end 20.0018 -9.41) (width 0.25) (layer "F.Cu") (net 5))
 (via (at 18.4658 -9.5504) (size 0.8) (drill 0.3) (layers "F.Cu" "B.Cu") (free) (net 5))
 (via (at 12.7254 -0.9906) (size 0.8) (drill 0.3) (layers "F.Cu" "B.Cu") (free) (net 5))
 (via (at 19.4564 -8.0518) (size 0.8) (drill 0.3) (layers "F.Cu" "B.Cu") (free) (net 5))
 (via (at 9.0678 -9.4488) (size 0.8) (drill 0.3) (layers "F.Cu" "B.Cu") (free) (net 5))
 (via (at 27.9146 -6.2738) (size 0.8) (drill 0.3) (layers "F.Cu" "B.Cu") (free) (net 5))
 (via (at 8.3058 -0.9398) (size 0.8) (drill 0.3) (layers "F.Cu" "B.Cu") (free) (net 5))
 (via (at 23.368 -1.905) (size 0.8) (drill 0.3) (layers "F.Cu" "B.Cu") (free) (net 5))
 (via (at 26.4668 -8.4074) (size 0.8) (drill 0.3) (layers "F.Cu" "B.Cu") (free) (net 5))
 (via (at 12.9794 -9.7028) (size 0.8) (drill 0.3) (layers "F.Cu" "B.Cu") (free) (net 5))
 (via (at 19.431 -1.905) (size 0.8) (drill 0.3) (layers "F.Cu" "B.Cu") (free) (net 5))
 (segment (start 2 -2.286) (end 5.824 -2.286) (width 0.25) (layer "F.Cu") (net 6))
 (segment (start 8.4074 -4.0132) (end 7.5512 -4.0132) (width 0.25) (layer "F.Cu") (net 6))
 (segment (start 6.57 -2.528) (end 6.318 -2.78) (width 0.25) (layer "F.Cu") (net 6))
 (segment (start 16.561 -8.787) (end 13.6892 -8.787) (width 0.25) (layer "F.Cu") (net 6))
 (segment (start 13.6892 -8.787) (end 11.42604 -6.52384) (width 0.25) (layer "F.Cu") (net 6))
 (segment (start 11.42604 -6.52384) (end 9.29244 -6.52384) (width 0.25) (layer "F.Cu") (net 6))
 (segment (start 9.62 -2.528) (end 6.57 -2.528) (width 0.25) (layer "F.Cu") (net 6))
 (segment (start 5.824 -2.286) (end 6.318 -2.78) (width 0.25) (layer "F.Cu") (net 6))
 (segment (start 7.5512 -4.0132) (end 6.318 -2.78) (width 0.25) (layer "F.Cu") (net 6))
 (segment (start 9.29244 -6.52384) (end 8.4328 -5.6642) (width 0.25) (layer "F.Cu") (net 6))
 (segment (start 18.236 -7.112) (end 16.561 -8.787) (width 0.25) (layer "F.Cu") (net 6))
 (via (at 8.4328 -5.6642) (size 0.8) (drill 0.3) (layers "F.Cu" "B.Cu") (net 6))
 (via (at 8.4074 -4.0132) (size 0.8) (drill 0.3) (layers "F.Cu" "B.Cu") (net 6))
 (segment (start 8.4328 -5.6642) (end 8.4328 -4.0386) (width 0.25) (layer "B.Cu") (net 6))
 (segment (start 8.4328 -4.0386) (end 8.4074 -4.0132) (width 0.25) (layer "B.Cu") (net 6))
 (segment (start 21.213 -9.41) (end 21.479 -9.144) (width 0.25) (layer "F.Cu") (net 7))
 (segment (start 21.479 -9.243) (end 19.812 -10.91) (width 0.25) (layer "F.Cu") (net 7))
 (segment (start 2.9652 -10.8712) (end 19.7732 -10.8712) (width 0.25) (layer "F.Cu") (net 7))
 (segment (start 31.486 -10.91) (end 32.48 -9.916) (width 0.25) (layer "F.Cu") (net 7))
 (segment (start 2 -9.906) (end 2.9652 -10.8712) (width 0.25) (layer "F.Cu") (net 7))
 (segment (start 19.7732 -10.8712) (end 19.812 -10.91) (width 0.25) (layer "F.Cu") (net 7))
 (segment (start 21.479 -9.144) (end 21.479 -9.243) (width 0.25) (layer "F.Cu") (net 7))
 (segment (start 19.812 -10.91) (end 31.486 -10.91) (width 0.25) (layer "F.Cu") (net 7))
 (segment (start 29.432 -5.854) (end 29.432 -4.318) (width 0.25) (layer "F.Cu") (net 3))
 (segment (start 32.48 -2.296) (end 30.4446 -2.296) (width 0.25) (layer "F.Cu") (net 3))
 (segment (start 30.4446 -2.296) (end 29.432 -3.3086) (width 0.25) (layer "F.Cu") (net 3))
 (segment (start 29.432 -3.3086) (end 29.432 -4.318) (width 0.25) (layer "F.Cu") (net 3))
 (segment (start 15.2842 -7.1882) (end 16.6598 -7.1882) (width 0.25) (layer "F.Cu") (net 4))
 (segment (start 20.32 -4.1148) (end 23.68636 -4.1148) (width 0.25) (layer "F.Cu") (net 4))
 (segment (start 14.192 -6.096) (end 15.2842 -7.1882) (width 0.25) (layer "F.Cu") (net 4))
 (segment (start 23.68636 -4.1148) (end 25.876 -1.92516) (width 0.25) (layer "F.Cu") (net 4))
 (segment (start 16.6598 -7.1882) (end 18.6664 -5.1816) (width 0.25) (layer "F.Cu") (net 4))
 (segment (start 26.75316 -1.048) (end 25.876 -1.92516) (width 0.25) (layer "F.Cu") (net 4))
 (segment (start 14.192 -7.135) (end 14.192 -6.096) (width 0.25) (layer "F.Cu") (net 4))
 (segment (start 18.6664 -5.1816) (end 19.1262 -5.1816) (width 0.25) (layer "F.Cu") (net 4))
 (segment (start 29.432 -1.048) (end 26.75316 -1.048) (width 0.25) (layer "F.Cu") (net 4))
 (via (at 19.1262 -5.1816) (size 0.8) (drill 0.3) (layers "F.Cu" "B.Cu") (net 4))
 (via (at 20.32 -4.1148) (size 0.8) (drill 0.3) (layers "F.Cu" "B.Cu") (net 4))
 (segment (start 19.2532 -5.1816) (end 20.32 -4.1148) (width 0.25) (layer "B.Cu") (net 4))
 (segment (start 19.1262 -5.1816) (end 19.2532 -5.1816) (width 0.25) (layer "B.Cu") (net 4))
 (segment (start 14.192 -3.071) (end 14.192 -1.778) (width 0.25) (layer "F.Cu") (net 2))
 (segment (start 14.192 -3.071) (end 14.513 -3.392) (width 0.25) (layer "F.Cu") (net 2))
 (segment (start 21.304 -6.21284) (end 21.81784 -6.21284) (width 0.25) (layer "F.Cu") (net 2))
 (segment (start 14.513 -3.392) (end 18.48316 -3.392) (width 0.25) (layer "F.Cu") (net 2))
 (segment (start 21.81784 -6.21284) (end 24.749 -9.144) (width 0.25) (layer "F.Cu") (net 2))
 (segment (start 18.48316 -3.392) (end 21.304 -6.21284) (width 0.25) (layer "F.Cu") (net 2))
 (segment (start 15.736 -8.062) (end 14.235 -8.062) (width 0.25) (layer "F.Cu") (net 10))
 (segment (start 14.235 -8.062) (end 14.192 -8.105) (width 0.25) (layer "F.Cu") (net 10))
 (segment (start 15.736 -4.602) (end 15.782 -4.556) (width 0.25) (layer "F.Cu") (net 9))
 (segment (start 15.736 -6.162) (end 15.736 -4.602) (width 0.25) (layer "F.Cu") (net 9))
 (segment (start 15.162 -1.778) (end 15.162 -2.4366) (width 0.25) (layer "F.Cu") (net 8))
 (segment (start 15.162 -2.4366) (end 15.3924 -2.667) (width 0.25) (layer "F.Cu") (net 8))
 (segment (start 16.781502 -4.3942) (end 17.5202 -4.3942) (width 0.25) (layer "F.Cu") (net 8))
 (segment (start 17.5202 -4.3942) (end 17.682 -4.556) (width 0.25) (layer "F.Cu") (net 8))
 (via (at 16.781502 -4.3942) (size 0.8) (drill 0.3) (layers "F.Cu" "B.Cu") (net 8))
 (via (at 15.3924 -2.667) (size 0.8) (drill 0.3) (layers "F.Cu" "B.Cu") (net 8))
 (segment (start 15.3924 -3.005098) (end 16.781502 -4.3942) (width 0.25) (layer "B.Cu") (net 8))
 (segment (start 15.3924 -2.667) (end 15.3924 -3.005098) (width 0.25) (layer "B.Cu") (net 8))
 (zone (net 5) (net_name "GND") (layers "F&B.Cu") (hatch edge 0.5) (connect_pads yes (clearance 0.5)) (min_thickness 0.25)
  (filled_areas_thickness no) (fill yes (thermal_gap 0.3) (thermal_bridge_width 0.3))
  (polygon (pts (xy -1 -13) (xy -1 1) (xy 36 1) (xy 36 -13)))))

